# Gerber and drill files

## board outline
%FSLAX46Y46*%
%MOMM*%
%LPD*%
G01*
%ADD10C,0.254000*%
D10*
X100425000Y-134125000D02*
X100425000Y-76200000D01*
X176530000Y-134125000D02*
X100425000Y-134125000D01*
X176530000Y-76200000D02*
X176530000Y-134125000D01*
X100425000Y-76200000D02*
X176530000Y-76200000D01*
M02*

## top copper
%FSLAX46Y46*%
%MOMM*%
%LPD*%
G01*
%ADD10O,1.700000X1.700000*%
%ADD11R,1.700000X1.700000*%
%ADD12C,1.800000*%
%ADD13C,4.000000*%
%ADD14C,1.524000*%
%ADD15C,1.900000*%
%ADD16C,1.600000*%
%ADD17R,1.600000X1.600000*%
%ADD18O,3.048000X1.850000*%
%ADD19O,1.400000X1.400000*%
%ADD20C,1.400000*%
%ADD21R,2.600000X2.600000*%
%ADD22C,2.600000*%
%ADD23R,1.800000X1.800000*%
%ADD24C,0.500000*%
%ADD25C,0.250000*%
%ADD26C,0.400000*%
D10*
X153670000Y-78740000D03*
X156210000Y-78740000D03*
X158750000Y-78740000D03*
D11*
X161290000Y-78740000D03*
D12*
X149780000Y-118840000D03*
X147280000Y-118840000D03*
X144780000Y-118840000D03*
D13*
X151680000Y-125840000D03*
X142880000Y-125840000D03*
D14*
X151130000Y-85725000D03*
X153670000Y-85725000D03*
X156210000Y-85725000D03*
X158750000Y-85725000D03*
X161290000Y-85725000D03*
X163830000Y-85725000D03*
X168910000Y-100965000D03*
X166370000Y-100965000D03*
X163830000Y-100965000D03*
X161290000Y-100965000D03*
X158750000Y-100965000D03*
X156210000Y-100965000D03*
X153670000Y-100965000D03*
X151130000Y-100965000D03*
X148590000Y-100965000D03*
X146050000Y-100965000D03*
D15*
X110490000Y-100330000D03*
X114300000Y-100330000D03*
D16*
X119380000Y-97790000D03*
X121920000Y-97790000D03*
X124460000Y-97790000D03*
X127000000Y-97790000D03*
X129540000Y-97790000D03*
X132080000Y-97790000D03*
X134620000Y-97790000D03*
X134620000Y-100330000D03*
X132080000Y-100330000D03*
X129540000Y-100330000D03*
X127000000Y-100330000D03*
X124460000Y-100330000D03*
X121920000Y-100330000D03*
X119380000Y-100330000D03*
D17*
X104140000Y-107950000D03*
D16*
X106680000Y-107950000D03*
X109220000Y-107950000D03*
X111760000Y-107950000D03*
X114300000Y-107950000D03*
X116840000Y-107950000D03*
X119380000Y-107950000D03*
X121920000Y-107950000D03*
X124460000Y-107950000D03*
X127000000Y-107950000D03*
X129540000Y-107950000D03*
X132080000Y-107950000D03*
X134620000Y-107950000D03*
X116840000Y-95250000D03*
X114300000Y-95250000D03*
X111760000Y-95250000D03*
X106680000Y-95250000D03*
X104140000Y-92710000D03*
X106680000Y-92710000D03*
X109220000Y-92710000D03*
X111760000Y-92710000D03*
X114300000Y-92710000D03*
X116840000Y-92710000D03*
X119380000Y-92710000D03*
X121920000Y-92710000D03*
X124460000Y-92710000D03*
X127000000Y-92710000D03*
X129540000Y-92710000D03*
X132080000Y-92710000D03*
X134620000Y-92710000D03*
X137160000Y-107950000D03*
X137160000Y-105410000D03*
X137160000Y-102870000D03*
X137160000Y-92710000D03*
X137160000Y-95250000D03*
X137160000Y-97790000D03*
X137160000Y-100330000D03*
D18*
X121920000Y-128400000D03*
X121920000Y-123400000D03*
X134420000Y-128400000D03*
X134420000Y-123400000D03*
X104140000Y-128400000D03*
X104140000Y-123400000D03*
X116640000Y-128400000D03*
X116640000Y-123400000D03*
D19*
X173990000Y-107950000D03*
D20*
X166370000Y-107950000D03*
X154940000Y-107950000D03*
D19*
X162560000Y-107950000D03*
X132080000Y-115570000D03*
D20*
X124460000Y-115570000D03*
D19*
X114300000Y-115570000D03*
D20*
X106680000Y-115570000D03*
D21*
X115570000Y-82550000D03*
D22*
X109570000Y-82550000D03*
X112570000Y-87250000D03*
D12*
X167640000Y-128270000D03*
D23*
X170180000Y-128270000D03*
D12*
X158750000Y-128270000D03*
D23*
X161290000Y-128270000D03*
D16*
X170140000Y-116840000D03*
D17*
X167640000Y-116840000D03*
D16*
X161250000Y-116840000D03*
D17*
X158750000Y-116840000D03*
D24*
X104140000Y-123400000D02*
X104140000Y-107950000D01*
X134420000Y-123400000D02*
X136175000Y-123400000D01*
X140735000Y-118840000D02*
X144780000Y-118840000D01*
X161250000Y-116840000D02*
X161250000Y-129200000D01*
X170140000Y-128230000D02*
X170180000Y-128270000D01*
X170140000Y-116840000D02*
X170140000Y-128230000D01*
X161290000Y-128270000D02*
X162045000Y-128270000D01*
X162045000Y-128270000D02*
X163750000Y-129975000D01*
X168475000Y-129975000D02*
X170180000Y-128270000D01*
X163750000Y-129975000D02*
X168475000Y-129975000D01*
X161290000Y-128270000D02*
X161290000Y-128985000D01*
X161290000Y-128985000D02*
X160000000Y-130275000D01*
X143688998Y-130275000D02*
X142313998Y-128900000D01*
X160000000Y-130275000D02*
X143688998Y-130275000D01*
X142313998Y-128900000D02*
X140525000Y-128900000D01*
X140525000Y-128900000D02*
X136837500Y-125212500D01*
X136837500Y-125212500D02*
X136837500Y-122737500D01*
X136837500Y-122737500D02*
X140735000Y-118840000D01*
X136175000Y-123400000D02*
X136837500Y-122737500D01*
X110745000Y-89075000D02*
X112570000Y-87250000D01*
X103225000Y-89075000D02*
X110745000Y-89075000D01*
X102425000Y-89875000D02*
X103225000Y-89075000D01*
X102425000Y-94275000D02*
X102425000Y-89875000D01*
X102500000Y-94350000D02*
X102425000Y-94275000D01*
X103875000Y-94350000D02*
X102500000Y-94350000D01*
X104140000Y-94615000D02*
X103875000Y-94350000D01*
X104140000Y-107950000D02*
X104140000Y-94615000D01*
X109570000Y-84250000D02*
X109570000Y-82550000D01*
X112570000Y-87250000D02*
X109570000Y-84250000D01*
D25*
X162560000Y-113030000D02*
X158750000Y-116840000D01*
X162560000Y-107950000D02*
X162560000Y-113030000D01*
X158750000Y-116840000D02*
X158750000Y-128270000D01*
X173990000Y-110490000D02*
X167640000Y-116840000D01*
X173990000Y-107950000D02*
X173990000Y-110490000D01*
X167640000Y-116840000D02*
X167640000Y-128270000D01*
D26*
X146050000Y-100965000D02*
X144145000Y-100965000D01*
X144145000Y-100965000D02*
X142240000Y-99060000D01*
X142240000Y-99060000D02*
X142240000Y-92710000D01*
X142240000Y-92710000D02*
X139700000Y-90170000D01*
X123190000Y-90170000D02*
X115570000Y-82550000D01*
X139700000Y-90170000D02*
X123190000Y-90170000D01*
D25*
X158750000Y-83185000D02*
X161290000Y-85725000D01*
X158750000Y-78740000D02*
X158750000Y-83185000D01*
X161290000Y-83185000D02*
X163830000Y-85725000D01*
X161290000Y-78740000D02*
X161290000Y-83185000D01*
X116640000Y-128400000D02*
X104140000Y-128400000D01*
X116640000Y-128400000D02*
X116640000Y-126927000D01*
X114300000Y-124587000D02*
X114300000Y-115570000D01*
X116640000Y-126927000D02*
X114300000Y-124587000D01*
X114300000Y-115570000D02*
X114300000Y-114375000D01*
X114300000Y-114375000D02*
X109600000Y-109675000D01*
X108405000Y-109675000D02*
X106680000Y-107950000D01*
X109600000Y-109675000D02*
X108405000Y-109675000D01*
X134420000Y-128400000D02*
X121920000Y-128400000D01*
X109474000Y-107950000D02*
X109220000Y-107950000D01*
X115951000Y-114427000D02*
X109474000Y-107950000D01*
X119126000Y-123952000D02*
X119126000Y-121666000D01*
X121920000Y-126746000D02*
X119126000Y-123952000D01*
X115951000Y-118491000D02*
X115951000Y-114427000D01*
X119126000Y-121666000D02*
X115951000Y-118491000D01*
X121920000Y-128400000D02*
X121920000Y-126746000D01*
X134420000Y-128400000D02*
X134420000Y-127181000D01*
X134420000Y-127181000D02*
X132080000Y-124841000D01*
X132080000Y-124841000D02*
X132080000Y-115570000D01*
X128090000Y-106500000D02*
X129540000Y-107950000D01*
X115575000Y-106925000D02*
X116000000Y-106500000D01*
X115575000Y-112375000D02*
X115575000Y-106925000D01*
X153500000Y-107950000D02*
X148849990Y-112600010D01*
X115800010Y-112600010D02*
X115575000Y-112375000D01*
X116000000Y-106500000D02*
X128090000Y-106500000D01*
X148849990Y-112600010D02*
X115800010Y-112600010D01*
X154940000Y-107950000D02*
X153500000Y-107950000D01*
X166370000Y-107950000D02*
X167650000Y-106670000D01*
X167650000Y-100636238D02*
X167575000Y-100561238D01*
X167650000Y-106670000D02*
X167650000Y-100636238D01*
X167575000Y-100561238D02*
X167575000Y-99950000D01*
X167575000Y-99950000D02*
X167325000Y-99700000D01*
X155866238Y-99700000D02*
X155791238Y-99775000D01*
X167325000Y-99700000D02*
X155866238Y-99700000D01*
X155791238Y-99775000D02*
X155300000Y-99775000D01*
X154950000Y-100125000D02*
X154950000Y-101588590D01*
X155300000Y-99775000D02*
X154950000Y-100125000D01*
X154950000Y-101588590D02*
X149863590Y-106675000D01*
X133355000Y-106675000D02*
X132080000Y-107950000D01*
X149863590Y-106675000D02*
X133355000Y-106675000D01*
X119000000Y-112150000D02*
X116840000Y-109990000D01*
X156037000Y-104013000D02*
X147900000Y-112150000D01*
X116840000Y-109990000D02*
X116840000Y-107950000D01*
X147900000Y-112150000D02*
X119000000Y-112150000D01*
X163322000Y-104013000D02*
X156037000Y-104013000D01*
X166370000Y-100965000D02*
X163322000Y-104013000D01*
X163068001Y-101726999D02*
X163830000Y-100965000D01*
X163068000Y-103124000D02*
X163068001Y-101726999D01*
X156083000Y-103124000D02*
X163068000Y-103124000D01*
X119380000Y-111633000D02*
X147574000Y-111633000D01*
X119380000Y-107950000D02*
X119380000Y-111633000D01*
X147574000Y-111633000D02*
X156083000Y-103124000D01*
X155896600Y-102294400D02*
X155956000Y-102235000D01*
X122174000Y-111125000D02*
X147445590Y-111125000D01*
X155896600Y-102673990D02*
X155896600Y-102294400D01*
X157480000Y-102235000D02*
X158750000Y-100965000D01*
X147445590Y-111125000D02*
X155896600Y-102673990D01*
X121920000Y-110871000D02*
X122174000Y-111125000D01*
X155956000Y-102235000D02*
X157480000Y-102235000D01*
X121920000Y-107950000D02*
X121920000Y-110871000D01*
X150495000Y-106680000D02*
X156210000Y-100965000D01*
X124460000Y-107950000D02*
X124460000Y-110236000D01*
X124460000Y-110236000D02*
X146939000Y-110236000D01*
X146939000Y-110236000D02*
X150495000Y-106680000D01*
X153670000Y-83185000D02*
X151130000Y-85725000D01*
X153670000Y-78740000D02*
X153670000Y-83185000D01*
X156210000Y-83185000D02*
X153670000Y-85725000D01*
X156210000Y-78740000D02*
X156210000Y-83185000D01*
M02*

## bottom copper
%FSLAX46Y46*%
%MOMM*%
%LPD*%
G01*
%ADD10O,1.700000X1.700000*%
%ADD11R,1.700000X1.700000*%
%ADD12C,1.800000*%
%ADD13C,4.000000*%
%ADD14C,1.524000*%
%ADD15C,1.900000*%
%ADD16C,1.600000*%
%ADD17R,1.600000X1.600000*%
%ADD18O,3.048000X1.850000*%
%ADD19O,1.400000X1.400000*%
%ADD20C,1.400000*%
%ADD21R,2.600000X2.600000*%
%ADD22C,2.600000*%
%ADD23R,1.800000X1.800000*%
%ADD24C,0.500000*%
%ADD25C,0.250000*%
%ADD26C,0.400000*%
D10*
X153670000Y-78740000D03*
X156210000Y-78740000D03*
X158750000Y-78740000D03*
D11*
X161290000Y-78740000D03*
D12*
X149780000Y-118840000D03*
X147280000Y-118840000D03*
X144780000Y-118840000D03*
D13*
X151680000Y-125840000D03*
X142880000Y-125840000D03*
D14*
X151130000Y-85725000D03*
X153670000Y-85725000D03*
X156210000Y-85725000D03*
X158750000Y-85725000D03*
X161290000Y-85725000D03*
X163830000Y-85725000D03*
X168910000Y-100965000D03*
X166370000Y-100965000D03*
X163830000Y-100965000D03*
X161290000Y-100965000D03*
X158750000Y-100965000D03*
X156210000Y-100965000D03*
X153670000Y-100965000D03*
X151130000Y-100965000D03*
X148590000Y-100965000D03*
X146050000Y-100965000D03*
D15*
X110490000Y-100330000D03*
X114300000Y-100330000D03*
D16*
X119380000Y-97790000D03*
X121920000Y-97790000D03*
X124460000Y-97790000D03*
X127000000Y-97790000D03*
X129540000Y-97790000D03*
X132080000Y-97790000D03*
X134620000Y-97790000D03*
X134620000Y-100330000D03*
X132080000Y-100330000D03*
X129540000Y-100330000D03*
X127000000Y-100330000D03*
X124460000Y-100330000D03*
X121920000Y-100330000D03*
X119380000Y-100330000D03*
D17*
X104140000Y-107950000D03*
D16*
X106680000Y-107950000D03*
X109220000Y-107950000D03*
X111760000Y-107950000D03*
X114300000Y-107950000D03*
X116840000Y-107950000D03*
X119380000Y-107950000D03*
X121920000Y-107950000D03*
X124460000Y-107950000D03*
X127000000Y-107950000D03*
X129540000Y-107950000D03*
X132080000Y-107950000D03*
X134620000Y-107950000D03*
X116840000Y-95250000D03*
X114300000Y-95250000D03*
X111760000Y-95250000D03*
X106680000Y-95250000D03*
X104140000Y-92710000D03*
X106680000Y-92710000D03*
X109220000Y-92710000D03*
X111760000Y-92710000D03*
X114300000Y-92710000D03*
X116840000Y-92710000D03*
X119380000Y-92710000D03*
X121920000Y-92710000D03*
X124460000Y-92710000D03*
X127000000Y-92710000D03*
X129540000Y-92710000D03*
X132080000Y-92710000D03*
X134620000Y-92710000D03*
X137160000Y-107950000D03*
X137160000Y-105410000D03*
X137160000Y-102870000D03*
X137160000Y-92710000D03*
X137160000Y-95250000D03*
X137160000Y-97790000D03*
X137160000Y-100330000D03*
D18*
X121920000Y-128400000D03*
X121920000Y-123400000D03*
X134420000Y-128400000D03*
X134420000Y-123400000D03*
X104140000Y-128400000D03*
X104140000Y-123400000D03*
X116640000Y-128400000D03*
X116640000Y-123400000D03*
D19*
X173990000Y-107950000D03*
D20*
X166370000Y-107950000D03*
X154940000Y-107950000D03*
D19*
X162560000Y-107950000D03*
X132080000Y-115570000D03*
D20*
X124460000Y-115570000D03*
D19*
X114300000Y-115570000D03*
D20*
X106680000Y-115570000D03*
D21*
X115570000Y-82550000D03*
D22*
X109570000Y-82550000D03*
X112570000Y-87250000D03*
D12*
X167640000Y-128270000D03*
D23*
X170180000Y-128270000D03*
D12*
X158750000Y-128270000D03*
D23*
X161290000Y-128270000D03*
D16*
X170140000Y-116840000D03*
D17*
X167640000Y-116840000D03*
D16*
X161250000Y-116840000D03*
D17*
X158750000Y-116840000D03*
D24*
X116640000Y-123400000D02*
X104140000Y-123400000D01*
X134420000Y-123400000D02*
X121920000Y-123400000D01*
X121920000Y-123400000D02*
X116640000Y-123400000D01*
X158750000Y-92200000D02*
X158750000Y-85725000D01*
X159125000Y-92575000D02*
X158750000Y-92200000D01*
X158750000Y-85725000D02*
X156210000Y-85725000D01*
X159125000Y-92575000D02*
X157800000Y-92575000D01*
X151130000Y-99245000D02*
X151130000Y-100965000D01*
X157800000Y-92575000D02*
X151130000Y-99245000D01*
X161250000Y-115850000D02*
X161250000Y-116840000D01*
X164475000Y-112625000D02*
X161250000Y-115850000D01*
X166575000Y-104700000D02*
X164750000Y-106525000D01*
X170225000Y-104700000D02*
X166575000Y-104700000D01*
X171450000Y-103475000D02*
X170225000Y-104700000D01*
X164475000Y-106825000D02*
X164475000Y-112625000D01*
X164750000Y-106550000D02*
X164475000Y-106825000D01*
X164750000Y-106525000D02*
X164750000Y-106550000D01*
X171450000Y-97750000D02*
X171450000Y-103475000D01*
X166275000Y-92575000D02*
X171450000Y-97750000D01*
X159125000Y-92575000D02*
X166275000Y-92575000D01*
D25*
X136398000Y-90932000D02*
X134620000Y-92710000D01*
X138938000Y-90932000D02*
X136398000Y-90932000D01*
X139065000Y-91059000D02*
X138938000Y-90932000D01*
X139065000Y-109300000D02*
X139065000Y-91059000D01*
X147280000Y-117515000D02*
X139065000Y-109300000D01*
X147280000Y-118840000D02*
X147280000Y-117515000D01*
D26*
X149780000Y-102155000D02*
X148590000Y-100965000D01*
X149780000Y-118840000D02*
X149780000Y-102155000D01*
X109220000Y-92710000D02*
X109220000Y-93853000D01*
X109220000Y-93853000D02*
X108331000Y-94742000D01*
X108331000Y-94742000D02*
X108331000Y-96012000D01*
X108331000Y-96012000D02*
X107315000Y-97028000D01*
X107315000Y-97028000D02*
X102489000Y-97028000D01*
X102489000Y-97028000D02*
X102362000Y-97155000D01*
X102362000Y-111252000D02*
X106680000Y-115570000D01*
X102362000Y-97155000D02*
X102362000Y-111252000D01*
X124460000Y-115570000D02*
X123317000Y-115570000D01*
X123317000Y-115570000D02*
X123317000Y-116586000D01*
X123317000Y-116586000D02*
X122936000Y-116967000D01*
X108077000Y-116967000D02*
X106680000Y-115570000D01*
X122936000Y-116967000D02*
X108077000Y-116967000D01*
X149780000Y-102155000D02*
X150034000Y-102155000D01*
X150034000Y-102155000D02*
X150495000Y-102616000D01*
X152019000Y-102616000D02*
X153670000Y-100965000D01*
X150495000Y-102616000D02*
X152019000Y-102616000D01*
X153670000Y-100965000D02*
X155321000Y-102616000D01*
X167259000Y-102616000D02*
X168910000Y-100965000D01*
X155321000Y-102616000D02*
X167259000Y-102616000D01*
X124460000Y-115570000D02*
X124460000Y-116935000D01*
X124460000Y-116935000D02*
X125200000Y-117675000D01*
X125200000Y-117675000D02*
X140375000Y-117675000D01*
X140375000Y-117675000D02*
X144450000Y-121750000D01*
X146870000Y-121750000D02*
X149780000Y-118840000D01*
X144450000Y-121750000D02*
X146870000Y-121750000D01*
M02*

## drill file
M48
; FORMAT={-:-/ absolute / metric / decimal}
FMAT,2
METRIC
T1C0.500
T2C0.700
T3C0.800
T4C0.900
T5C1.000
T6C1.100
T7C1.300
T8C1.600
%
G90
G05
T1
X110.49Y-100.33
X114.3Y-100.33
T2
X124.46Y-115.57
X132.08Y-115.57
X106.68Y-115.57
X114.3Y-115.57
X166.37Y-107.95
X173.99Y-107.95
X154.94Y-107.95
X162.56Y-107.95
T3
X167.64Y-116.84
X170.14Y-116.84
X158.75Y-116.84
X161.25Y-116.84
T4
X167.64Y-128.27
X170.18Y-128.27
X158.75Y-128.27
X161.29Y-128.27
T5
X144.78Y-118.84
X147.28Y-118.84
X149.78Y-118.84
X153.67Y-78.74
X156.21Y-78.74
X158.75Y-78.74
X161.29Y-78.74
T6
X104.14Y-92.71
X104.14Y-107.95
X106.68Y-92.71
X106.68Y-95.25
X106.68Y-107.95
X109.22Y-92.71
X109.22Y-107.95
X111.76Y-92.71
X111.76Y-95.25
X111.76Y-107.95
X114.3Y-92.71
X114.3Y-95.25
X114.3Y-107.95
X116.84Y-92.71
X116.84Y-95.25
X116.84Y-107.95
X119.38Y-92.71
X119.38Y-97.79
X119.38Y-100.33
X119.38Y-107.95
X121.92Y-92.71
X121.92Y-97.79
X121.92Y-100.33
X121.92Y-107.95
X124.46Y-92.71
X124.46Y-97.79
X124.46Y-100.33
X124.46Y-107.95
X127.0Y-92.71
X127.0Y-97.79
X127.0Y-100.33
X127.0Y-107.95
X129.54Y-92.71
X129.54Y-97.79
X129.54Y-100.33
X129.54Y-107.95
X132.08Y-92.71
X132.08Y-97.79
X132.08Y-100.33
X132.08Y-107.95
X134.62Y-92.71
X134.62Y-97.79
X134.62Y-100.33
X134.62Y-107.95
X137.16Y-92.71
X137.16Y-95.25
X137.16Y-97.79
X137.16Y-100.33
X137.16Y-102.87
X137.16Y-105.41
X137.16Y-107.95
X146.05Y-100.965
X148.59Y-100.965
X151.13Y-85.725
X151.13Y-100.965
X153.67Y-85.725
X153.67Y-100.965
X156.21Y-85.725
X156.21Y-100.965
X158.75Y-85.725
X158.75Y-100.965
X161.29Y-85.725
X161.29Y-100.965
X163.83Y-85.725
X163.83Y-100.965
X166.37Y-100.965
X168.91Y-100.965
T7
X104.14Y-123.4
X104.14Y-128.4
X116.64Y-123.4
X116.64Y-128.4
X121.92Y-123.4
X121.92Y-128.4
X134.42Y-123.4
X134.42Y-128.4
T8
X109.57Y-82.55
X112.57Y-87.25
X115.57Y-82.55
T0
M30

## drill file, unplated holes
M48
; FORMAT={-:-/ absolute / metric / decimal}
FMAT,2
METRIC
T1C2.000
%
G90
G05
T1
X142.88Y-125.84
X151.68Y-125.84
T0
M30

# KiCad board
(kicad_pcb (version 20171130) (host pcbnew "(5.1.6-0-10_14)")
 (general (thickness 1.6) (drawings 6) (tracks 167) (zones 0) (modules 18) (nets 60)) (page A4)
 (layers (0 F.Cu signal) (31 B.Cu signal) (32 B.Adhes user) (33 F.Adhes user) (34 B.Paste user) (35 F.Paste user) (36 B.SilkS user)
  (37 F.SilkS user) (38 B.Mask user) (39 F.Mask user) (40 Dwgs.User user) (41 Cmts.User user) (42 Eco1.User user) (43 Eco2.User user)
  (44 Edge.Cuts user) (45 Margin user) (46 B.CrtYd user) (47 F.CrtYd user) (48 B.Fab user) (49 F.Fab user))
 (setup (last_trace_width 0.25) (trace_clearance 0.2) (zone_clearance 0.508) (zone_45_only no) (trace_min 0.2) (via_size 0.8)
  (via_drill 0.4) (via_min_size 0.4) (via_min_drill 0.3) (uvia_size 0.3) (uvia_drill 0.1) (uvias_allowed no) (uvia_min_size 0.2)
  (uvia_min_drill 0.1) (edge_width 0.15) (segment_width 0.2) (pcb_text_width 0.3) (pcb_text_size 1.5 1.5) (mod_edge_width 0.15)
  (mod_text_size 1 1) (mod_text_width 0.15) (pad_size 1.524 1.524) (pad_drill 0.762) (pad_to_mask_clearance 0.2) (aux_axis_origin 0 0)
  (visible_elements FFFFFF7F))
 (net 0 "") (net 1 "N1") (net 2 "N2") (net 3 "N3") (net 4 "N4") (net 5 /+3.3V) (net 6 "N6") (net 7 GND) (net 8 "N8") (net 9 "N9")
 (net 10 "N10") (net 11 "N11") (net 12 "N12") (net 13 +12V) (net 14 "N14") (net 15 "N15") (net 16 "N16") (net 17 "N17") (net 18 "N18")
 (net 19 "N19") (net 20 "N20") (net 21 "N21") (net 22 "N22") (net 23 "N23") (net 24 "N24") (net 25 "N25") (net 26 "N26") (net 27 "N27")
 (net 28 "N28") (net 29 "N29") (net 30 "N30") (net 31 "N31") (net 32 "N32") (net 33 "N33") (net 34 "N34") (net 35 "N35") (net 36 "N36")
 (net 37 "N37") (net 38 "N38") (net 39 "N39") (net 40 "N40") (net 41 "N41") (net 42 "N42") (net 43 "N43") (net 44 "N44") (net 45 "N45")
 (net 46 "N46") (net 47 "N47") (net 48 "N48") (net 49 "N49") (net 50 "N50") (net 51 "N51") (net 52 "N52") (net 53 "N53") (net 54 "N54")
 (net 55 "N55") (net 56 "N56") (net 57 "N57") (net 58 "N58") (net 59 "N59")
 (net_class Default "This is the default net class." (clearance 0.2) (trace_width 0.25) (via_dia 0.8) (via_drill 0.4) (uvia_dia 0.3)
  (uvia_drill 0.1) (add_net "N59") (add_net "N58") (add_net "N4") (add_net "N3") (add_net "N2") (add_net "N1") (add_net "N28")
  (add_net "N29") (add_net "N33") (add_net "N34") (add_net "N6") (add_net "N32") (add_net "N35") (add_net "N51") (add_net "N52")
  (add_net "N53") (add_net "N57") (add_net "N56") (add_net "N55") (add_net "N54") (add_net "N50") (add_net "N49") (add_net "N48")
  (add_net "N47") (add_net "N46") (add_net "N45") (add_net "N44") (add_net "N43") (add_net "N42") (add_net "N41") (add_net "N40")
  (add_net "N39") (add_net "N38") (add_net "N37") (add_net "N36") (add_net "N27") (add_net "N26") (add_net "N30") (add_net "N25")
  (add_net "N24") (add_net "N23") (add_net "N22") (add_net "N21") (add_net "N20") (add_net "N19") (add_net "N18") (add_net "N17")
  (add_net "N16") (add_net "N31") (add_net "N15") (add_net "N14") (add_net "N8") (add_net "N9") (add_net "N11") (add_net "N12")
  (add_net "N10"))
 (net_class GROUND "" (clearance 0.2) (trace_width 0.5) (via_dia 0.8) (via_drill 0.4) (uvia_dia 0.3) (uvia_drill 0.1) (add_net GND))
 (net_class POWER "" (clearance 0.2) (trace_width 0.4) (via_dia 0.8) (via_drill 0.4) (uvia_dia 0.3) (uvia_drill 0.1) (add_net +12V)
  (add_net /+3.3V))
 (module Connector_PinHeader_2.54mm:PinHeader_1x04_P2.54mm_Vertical (layer F.Cu) (at 161.29 78.74 270)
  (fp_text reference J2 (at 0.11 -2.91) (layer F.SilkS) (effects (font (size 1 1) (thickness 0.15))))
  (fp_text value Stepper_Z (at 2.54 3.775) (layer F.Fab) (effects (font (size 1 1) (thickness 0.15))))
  (pad 4 thru_hole oval (at 0 7.62 270) (size 1.7 1.7) (drill 1) (layers *.Cu *.Mask) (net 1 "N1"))
  (pad 3 thru_hole oval (at 0 5.08 270) (size 1.7 1.7) (drill 1) (layers *.Cu *.Mask) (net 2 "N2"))
  (pad 2 thru_hole oval (at 0 2.54 270) (size 1.7 1.7) (drill 1) (layers *.Cu *.Mask) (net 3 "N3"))
  (pad 1 thru_hole rect (at 0 0 270) (size 1.7 1.7) (drill 1) (layers *.Cu *.Mask) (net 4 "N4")))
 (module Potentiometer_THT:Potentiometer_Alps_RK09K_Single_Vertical (layer F.Cu) (at 144.78 118.84 270)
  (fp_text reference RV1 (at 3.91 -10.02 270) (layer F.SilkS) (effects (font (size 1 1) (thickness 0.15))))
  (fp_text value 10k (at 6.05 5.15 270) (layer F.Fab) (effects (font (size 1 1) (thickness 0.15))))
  (pad 3 thru_hole circle (at 0 -5 270) (size 1.8 1.8) (drill 1) (layers *.Cu *.Mask) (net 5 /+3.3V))
  (pad 2 thru_hole circle (at 0 -2.5 270) (size 1.8 1.8) (drill 1) (layers *.Cu *.Mask) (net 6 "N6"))
  (pad 1 thru_hole circle (at 0 0 270) (size 1.8 1.8) (drill 1) (layers *.Cu *.Mask) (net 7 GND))
  (pad "" np_thru_hole circle (at 7 -6.9 270) (size 4 4) (drill 2) (layers *.Cu *.Mask))
  (pad "" np_thru_hole circle (at 7 1.9 270) (size 4 4) (drill 2) (layers *.Cu *.Mask)))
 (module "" (layer F.Cu) (at 149.86 129.54)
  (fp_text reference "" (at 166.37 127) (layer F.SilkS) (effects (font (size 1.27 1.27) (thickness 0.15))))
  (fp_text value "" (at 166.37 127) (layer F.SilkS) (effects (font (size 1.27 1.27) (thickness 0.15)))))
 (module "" (layer F.Cu) (at 166.37 127)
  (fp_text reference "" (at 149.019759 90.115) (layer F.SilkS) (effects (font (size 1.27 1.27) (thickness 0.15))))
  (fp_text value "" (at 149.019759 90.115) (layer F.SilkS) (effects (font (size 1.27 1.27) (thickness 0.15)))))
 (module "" (layer F.Cu) (at 148.59 127)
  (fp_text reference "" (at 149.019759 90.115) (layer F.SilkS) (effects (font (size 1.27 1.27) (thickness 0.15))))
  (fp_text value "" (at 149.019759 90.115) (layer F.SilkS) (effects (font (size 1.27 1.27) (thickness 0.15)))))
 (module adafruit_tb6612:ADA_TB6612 (layer F.Cu) (at 157.48 93.98 90)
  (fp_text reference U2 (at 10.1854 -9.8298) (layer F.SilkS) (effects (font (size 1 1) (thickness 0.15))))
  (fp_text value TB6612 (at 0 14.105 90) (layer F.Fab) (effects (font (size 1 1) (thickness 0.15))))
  (pad 16 thru_hole circle (at 8.255 -6.35 90) (size 1.524 1.524) (drill 1.1) (layers *.Cu *.Mask) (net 1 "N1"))
  (pad 15 thru_hole circle (at 8.255 -3.81 90) (size 1.524 1.524) (drill 1.1) (layers *.Cu *.Mask) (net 2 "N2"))
  (pad 14 thru_hole circle (at 8.255 -1.27 90) (size 1.524 1.524) (drill 1.1) (layers *.Cu *.Mask) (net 7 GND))
  (pad 13 thru_hole circle (at 8.255 1.27 90) (size 1.524 1.524) (drill 1.1) (layers *.Cu *.Mask) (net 7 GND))
  (pad 12 thru_hole circle (at 8.255 3.81 90) (size 1.524 1.524) (drill 1.1) (layers *.Cu *.Mask) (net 3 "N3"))
  (pad 11 thru_hole circle (at 8.255 6.35 90) (size 1.524 1.524) (drill 1.1) (layers *.Cu *.Mask) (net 4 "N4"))
  (pad 10 thru_hole circle (at -6.985 11.43 90) (size 1.524 1.524) (drill 1.1) (layers *.Cu *.Mask) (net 5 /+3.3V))
  (pad 9 thru_hole circle (at -6.985 8.89 90) (size 1.524 1.524) (drill 1.1) (layers *.Cu *.Mask) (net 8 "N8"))
  (pad 8 thru_hole circle (at -6.985 6.35 90) (size 1.524 1.524) (drill 1.1) (layers *.Cu *.Mask) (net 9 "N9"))
  (pad 7 thru_hole circle (at -6.985 3.81 90) (size 1.524 1.524) (drill 1.1) (layers *.Cu *.Mask) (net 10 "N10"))
  (pad 6 thru_hole circle (at -6.985 1.27 90) (size 1.524 1.524) (drill 1.1) (layers *.Cu *.Mask) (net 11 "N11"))
  (pad 5 thru_hole circle (at -6.985 -1.27 90) (size 1.524 1.524) (drill 1.1) (layers *.Cu *.Mask) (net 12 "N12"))
  (pad 4 thru_hole circle (at -6.985 -3.81 90) (size 1.524 1.524) (drill 1.1) (layers *.Cu *.Mask) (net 5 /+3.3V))
  (pad 3 thru_hole circle (at -6.985 -6.35 90) (size 1.524 1.524) (drill 1.1) (layers *.Cu *.Mask) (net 7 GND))
  (pad 2 thru_hole circle (at -6.985 -8.89 90) (size 1.524 1.524) (drill 1.1) (layers *.Cu *.Mask) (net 5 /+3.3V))
  (pad 1 thru_hole circle (at -6.985 -11.43 90) (size 1.524 1.524) (drill 1.1) (layers *.Cu *.Mask) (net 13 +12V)))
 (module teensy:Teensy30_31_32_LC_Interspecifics (layer F.Cu) (at 120.65 100.33)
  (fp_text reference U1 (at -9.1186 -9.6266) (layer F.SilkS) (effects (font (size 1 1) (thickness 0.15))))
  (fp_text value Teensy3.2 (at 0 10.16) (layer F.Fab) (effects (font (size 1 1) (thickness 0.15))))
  (pad 52 thru_hole circle (at -10.16 0) (size 1.9 1.9) (drill 0.5) (layers *.Cu *.Mask F.SilkS))
  (pad 52 thru_hole circle (at -6.35 0) (size 1.9 1.9) (drill 0.5) (layers *.Cu *.Mask F.SilkS))
  (pad 51 thru_hole circle (at -1.27 -2.54) (size 1.6 1.6) (drill 1.1) (layers *.Cu *.Mask) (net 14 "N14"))
  (pad 50 thru_hole circle (at 1.27 -2.54) (size 1.6 1.6) (drill 1.1) (layers *.Cu *.Mask) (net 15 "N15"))
  (pad 49 thru_hole circle (at 3.81 -2.54) (size 1.6 1.6) (drill 1.1) (layers *.Cu *.Mask) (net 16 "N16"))
  (pad 48 thru_hole circle (at 6.35 -2.54) (size 1.6 1.6) (drill 1.1) (layers *.Cu *.Mask) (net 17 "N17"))
  (pad 47 thru_hole circle (at 8.89 -2.54) (size 1.6 1.6) (drill 1.1) (layers *.Cu *.Mask) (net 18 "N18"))
  (pad 46 thru_hole circle (at 11.43 -2.54) (size 1.6 1.6) (drill 1.1) (layers *.Cu *.Mask) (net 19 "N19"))
  (pad 45 thru_hole circle (at 13.97 -2.54) (size 1.6 1.6) (drill 1.1) (layers *.Cu *.Mask) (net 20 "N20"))
  (pad 44 thru_hole circle (at 13.97 0) (size 1.6 1.6) (drill 1.1) (layers *.Cu *.Mask) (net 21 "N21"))
  (pad 43 thru_hole circle (at 11.43 0) (size 1.6 1.6) (drill 1.1) (layers *.Cu *.Mask) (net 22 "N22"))
  (pad 42 thru_hole circle (at 8.89 0) (size 1.6 1.6) (drill 1.1) (layers *.Cu *.Mask) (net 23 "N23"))
  (pad 41 thru_hole circle (at 6.35 0) (size 1.6 1.6) (drill 1.1) (layers *.Cu *.Mask) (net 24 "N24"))
  (pad 40 thru_hole circle (at 3.81 0) (size 1.6 1.6) (drill 1.1) (layers *.Cu *.Mask) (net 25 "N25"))
  (pad 39 thru_hole circle (at 1.27 0) (size 1.6 1.6) (drill 1.1) (layers *.Cu *.Mask) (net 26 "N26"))
  (pad 38 thru_hole circle (at -1.27 0) (size 1.6 1.6) (drill 1.1) (layers *.Cu *.Mask) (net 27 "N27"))
  (pad 1 thru_hole rect (at -16.51 7.62) (size 1.6 1.6) (drill 1.1) (layers *.Cu *.Mask F.SilkS) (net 7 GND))
  (pad 2 thru_hole circle (at -13.97 7.62) (size 1.6 1.6) (drill 1.1) (layers *.Cu *.Mask F.SilkS) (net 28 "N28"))
  (pad 3 thru_hole circle (at -11.43 7.62) (size 1.6 1.6) (drill 1.1) (layers *.Cu *.Mask F.SilkS) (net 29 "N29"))
  (pad 4 thru_hole circle (at -8.89 7.62) (size 1.6 1.6) (drill 1.1) (layers *.Cu *.Mask F.SilkS) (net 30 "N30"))
  (pad 5 thru_hole circle (at -6.35 7.62) (size 1.6 1.6) (drill 1.1) (layers *.Cu *.Mask F.SilkS) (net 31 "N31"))
  (pad 6 thru_hole circle (at -3.81 7.62) (size 1.6 1.6) (drill 1.1) (layers *.Cu *.Mask F.SilkS) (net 8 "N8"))
  (pad 7 thru_hole circle (at -1.27 7.62) (size 1.6 1.6) (drill 1.1) (layers *.Cu *.Mask F.SilkS) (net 9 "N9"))
  (pad 8 thru_hole circle (at 1.27 7.62) (size 1.6 1.6) (drill 1.1) (layers *.Cu *.Mask F.SilkS) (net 11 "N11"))
  (pad 9 thru_hole circle (at 3.81 7.62) (size 1.6 1.6) (drill 1.1) (layers *.Cu *.Mask F.SilkS) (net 12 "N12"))
  (pad 10 thru_hole circle (at 6.35 7.62) (size 1.6 1.6) (drill 1.1) (layers *.Cu *.Mask F.SilkS) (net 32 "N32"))
  (pad 11 thru_hole circle (at 8.89 7.62) (size 1.6 1.6) (drill 1.1) (layers *.Cu *.Mask F.SilkS) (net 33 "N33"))
  (pad 12 thru_hole circle (at 11.43 7.62) (size 1.6 1.6) (drill 1.1) (layers *.Cu *.Mask F.SilkS) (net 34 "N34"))
  (pad 13 thru_hole circle (at 13.97 7.62) (size 1.6 1.6) (drill 1.1) (layers *.Cu *.Mask F.SilkS) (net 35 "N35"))
  (pad 37 thru_hole circle (at -3.81 -5.08) (size 1.6 1.6) (drill 1.1) (layers *.Cu *.Mask F.SilkS) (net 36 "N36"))
  (pad 36 thru_hole circle (at -6.35 -5.08) (size 1.6 1.6) (drill 1.1) (layers *.Cu *.Mask F.SilkS) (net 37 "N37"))
  (pad 35 thru_hole circle (at -8.89 -5.08) (size 1.6 1.6) (drill 1.1) (layers *.Cu *.Mask F.SilkS) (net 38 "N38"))
  (pad 34 thru_hole circle (at -13.97 -5.08) (size 1.6 1.6) (drill 1.1) (layers *.Cu *.Mask F.SilkS) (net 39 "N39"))
  (pad 33 thru_hole circle (at -16.51 -7.62) (size 1.6 1.6) (drill 1.1) (layers *.Cu *.Mask F.SilkS) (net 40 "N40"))
  (pad 32 thru_hole circle (at -13.97 -7.62) (size 1.6 1.6) (drill 1.1) (layers *.Cu *.Mask F.SilkS) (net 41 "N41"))
  (pad 31 thru_hole circle (at -11.43 -7.62) (size 1.6 1.6) (drill 1.1) (layers *.Cu *.Mask F.SilkS) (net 5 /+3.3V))
  (pad 30 thru_hole circle (at -8.89 -7.62) (size 1.6 1.6) (drill 1.1) (layers *.Cu *.Mask F.SilkS) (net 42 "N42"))
  (pad 29 thru_hole circle (at -6.35 -7.62) (size 1.6 1.6) (drill 1.1) (layers *.Cu *.Mask F.SilkS) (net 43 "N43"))
  (pad 28 thru_hole circle (at -3.81 -7.62) (size 1.6 1.6) (drill 1.1) (layers *.Cu *.Mask F.SilkS) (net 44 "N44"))
  (pad 27 thru_hole circle (at -1.27 -7.62) (size 1.6 1.6) (drill 1.1) (layers *.Cu *.Mask F.SilkS) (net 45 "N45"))
  (pad 26 thru_hole circle (at 1.27 -7.62) (size 1.6 1.6) (drill 1.1) (layers *.Cu *.Mask F.SilkS) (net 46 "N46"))
  (pad 25 thru_hole circle (at 3.81 -7.62) (size 1.6 1.6) (drill 1.1) (layers *.Cu *.Mask F.SilkS) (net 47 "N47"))
  (pad 24 thru_hole circle (at 6.35 -7.62) (size 1.6 1.6) (drill 1.1) (layers *.Cu *.Mask F.SilkS) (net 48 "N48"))
  (pad 23 thru_hole circle (at 8.89 -7.62) (size 1.6 1.6) (drill 1.1) (layers *.Cu *.Mask F.SilkS) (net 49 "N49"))
  (pad 22 thru_hole circle (at 11.43 -7.62) (size 1.6 1.6) (drill 1.1) (layers *.Cu *.Mask F.SilkS) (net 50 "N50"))
  (pad 21 thru_hole circle (at 13.97 -7.62) (size 1.6 1.6) (drill 1.1) (layers *.Cu *.Mask F.SilkS) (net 6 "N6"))
  (pad 14 thru_hole circle (at 16.51 7.62) (size 1.6 1.6) (drill 1.1) (layers *.Cu *.Mask F.SilkS) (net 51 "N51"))
  (pad 15 thru_hole circle (at 16.51 5.08) (size 1.6 1.6) (drill 1.1) (layers *.Cu *.Mask F.SilkS) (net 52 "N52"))
  (pad 16 thru_hole circle (at 16.51 2.54) (size 1.6 1.6) (drill 1.1) (layers *.Cu *.Mask F.SilkS) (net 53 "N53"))
  (pad 20 thru_hole circle (at 16.51 -7.62) (size 1.6 1.6) (drill 1.1) (layers *.Cu *.Mask F.SilkS) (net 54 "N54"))
  (pad 19 thru_hole circle (at 16.51 -5.08) (size 1.6 1.6) (drill 1.1) (layers *.Cu *.Mask F.SilkS) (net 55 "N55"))
  (pad 18 thru_hole circle (at 16.51 -2.54) (size 1.6 1.6) (drill 1.1) (layers *.Cu *.Mask F.SilkS) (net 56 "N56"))
  (pad 17 thru_hole circle (at 16.51 0) (size 1.6 1.6) (drill 1.1) (layers *.Cu *.Mask F.SilkS) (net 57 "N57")))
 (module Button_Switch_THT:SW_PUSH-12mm (layer F.Cu) (at 121.92 123.4)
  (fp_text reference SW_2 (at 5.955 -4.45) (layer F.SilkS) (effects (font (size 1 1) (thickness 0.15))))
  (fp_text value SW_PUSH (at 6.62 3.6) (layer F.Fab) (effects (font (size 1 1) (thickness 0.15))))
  (pad 2 thru_hole oval (at 0 5) (size 3.048 1.85) (drill 1.3) (layers *.Cu *.Mask) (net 29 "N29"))
  (pad 1 thru_hole oval (at 0 0) (size 3.048 1.85) (drill 1.3) (layers *.Cu *.Mask) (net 7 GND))
  (pad 2 thru_hole oval (at 12.5 5) (size 3.048 1.85) (drill 1.3) (layers *.Cu *.Mask) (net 29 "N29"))
  (pad 1 thru_hole oval (at 12.5 0) (size 3.048 1.85) (drill 1.3) (layers *.Cu *.Mask) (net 7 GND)))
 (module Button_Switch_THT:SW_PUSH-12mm (layer F.Cu) (at 104.14 123.4)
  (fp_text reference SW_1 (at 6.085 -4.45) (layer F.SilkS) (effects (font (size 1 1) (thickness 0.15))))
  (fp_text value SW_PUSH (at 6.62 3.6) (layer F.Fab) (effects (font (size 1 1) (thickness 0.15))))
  (pad 2 thru_hole oval (at 0 5) (size 3.048 1.85) (drill 1.3) (layers *.Cu *.Mask) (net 28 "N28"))
  (pad 1 thru_hole oval (at 0 0) (size 3.048 1.85) (drill 1.3) (layers *.Cu *.Mask) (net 7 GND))
  (pad 2 thru_hole oval (at 12.5 5) (size 3.048 1.85) (drill 1.3) (layers *.Cu *.Mask) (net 28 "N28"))
  (pad 1 thru_hole oval (at 12.5 0) (size 3.048 1.85) (drill 1.3) (layers *.Cu *.Mask) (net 7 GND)))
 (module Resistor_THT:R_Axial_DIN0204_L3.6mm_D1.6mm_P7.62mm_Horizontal (layer F.Cu) (at 166.37 107.95)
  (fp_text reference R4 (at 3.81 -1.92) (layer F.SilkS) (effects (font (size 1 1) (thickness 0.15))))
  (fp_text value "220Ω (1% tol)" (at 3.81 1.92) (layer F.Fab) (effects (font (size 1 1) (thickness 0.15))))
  (pad 2 thru_hole oval (at 7.62 0) (size 1.4 1.4) (drill 0.7) (layers *.Cu *.Mask) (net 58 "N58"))
  (pad 1 thru_hole circle (at 0 0) (size 1.4 1.4) (drill 0.7) (layers *.Cu *.Mask) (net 34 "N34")))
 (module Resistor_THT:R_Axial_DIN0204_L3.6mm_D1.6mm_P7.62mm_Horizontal (layer F.Cu) (at 154.94 107.95)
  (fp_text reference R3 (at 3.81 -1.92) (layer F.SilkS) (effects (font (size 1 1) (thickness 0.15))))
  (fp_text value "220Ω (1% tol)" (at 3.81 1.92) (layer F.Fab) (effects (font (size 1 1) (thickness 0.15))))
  (pad 1 thru_hole circle (at 0 0) (size 1.4 1.4) (drill 0.7) (layers *.Cu *.Mask) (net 33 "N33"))
  (pad 2 thru_hole oval (at 7.62 0) (size 1.4 1.4) (drill 0.7) (layers *.Cu *.Mask) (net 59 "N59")))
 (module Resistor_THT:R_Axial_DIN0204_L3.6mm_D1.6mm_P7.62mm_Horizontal (layer F.Cu) (at 124.46 115.57)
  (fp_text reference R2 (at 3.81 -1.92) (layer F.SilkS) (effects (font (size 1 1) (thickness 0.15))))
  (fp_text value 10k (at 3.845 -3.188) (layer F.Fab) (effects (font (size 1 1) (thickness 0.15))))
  (pad 2 thru_hole oval (at 7.62 0) (size 1.4 1.4) (drill 0.7) (layers *.Cu *.Mask) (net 29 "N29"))
  (pad 1 thru_hole circle (at 0 0) (size 1.4 1.4) (drill 0.7) (layers *.Cu *.Mask) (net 5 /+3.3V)))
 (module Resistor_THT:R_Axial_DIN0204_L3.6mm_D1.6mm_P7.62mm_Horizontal (layer F.Cu) (at 106.68 115.57)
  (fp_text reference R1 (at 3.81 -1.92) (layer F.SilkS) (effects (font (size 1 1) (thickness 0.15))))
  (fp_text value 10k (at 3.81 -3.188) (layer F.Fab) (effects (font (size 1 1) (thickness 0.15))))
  (pad 2 thru_hole oval (at 7.62 0) (size 1.4 1.4) (drill 0.7) (layers *.Cu *.Mask) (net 28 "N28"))
  (pad 1 thru_hole circle (at 0 0) (size 1.4 1.4) (drill 0.7) (layers *.Cu *.Mask) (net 5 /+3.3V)))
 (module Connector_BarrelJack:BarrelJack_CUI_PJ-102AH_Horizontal (layer F.Cu) (at 115.57 82.55 270)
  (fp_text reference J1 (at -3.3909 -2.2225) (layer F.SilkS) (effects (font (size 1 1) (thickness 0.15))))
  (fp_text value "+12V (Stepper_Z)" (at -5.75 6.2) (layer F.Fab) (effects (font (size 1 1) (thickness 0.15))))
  (pad 1 thru_hole rect (at 0 0 270) (size 2.6 2.6) (drill 1.6) (layers *.Cu *.Mask) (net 13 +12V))
  (pad 2 thru_hole circle (at 0 6 270) (size 2.6 2.6) (drill 1.6) (layers *.Cu *.Mask) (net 7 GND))
  (pad 3 thru_hole circle (at 4.7 3 270) (size 2.6 2.6) (drill 1.6) (layers *.Cu *.Mask) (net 7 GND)))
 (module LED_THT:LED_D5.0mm (layer F.Cu) (at 170.18 128.27 180)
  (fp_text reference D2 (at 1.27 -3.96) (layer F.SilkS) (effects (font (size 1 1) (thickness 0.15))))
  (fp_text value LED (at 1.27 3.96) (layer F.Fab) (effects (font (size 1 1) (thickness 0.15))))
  (pad 2 thru_hole circle (at 2.54 0 180) (size 1.8 1.8) (drill 0.9) (layers *.Cu *.Mask) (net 58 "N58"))
  (pad 1 thru_hole rect (at 0 0 180) (size 1.8 1.8) (drill 0.9) (layers *.Cu *.Mask) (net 7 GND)))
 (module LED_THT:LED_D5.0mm (layer F.Cu) (at 161.29 128.27 180)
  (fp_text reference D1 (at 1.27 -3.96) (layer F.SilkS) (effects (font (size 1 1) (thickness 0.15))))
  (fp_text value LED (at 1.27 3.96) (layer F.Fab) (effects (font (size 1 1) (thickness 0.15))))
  (pad 2 thru_hole circle (at 2.54 0 180) (size 1.8 1.8) (drill 0.9) (layers *.Cu *.Mask) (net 59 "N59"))
  (pad 1 thru_hole rect (at 0 0 180) (size 1.8 1.8) (drill 0.9) (layers *.Cu *.Mask) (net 7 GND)))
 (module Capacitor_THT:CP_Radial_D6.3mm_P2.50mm (layer F.Cu) (at 167.64 116.84)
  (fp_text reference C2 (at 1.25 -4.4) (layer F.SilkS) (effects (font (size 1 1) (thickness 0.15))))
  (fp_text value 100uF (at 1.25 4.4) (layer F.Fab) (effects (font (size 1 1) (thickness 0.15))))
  (pad 2 thru_hole circle (at 2.5 0) (size 1.6 1.6) (drill 0.8) (layers *.Cu *.Mask) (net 7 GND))
  (pad 1 thru_hole rect (at 0 0) (size 1.6 1.6) (drill 0.8) (layers *.Cu *.Mask) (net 58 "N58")))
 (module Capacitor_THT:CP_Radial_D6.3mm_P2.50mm (layer F.Cu) (at 158.75 116.84)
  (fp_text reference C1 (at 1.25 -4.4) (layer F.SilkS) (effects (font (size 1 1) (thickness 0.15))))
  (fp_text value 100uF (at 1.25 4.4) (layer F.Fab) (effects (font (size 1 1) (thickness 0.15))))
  (pad 2 thru_hole circle (at 2.5 0) (size 1.6 1.6) (drill 0.8) (layers *.Cu *.Mask) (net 7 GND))
  (pad 1 thru_hole rect (at 0 0) (size 1.6 1.6) (drill 0.8) (layers *.Cu *.Mask) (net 59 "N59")))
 (gr_line (start 100.425 134.125) (end 100.425 76.2) (layer Edge.Cuts) (width 0.254))
 (gr_line (start 176.53 134.125) (end 100.425 134.125) (layer Edge.Cuts) (width 0.254))
 (gr_line (start 176.53 76.2) (end 176.53 134.125) (layer Edge.Cuts) (width 0.254))
 (gr_line (start 100.425 76.2) (end 176.53 76.2) (layer Edge.Cuts) (width 0.254))
 (segment (start 104.14 123.4) (end 104.14 107.95) (width 0.5) (layer F.Cu) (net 7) (status 30))
 (segment (start 116.64 123.4) (end 104.14 123.4) (width 0.5) (layer B.Cu) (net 7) (status 30))
 (segment (start 134.42 123.4) (end 121.92 123.4) (width 0.5) (layer B.Cu) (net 7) (status 30))
 (segment (start 121.92 123.4) (end 116.64 123.4) (width 0.5) (layer B.Cu) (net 7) (status 30))
 (segment (start 134.42 123.4) (end 136.175 123.4) (width 0.5) (layer F.Cu) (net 7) (status 10))
 (segment (start 140.735 118.84) (end 144.78 118.84) (width 0.5) (layer F.Cu) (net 7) (status 20))
 (segment (start 161.25 116.84) (end 161.25 129.2) (width 0.5) (layer F.Cu) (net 7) (status 10))
 (segment (start 170.14 128.23) (end 170.18 128.27) (width 0.5) (layer F.Cu) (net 7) (status 30))
 (segment (start 170.14 116.84) (end 170.14 128.23) (width 0.5) (layer F.Cu) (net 7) (status 30))
 (segment (start 161.29 128.27) (end 162.045 128.27) (width 0.5) (layer F.Cu) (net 7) (status 30))
 (segment (start 162.045 128.27) (end 163.75 129.975) (width 0.5) (layer F.Cu) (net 7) (status 10))
 (segment (start 168.475 129.975) (end 170.18 128.27) (width 0.5) (layer F.Cu) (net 7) (status 20))
 (segment (start 163.75 129.975) (end 168.475 129.975) (width 0.5) (layer F.Cu) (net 7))
 (segment (start 158.75 92.2) (end 158.75 85.725) (width 0.5) (layer B.Cu) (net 7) (status 20))
 (segment (start 159.125 92.575) (end 158.75 92.2) (width 0.5) (layer B.Cu) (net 7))
 (segment (start 158.75 85.725) (end 156.21 85.725) (width 0.5) (layer B.Cu) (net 7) (status 30))
 (segment (start 159.125 92.575) (end 157.8 92.575) (width 0.5) (layer B.Cu) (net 7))
 (segment (start 151.13 99.245) (end 151.13 100.965) (width 0.5) (layer B.Cu) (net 7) (status 20))
 (segment (start 157.8 92.575) (end 151.13 99.245) (width 0.5) (layer B.Cu) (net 7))
 (segment (start 161.29 128.27) (end 161.29 128.985) (width 0.5) (layer F.Cu) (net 7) (status 30))
 (segment (start 161.29 128.985) (end 160 130.275) (width 0.5) (layer F.Cu) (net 7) (status 10))
 (segment (start 143.688998 130.275) (end 142.313998 128.9) (width 0.5) (layer F.Cu) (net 7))
 (segment (start 160 130.275) (end 143.688998 130.275) (width 0.5) (layer F.Cu) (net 7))
 (segment (start 142.313998 128.9) (end 140.525 128.9) (width 0.5) (layer F.Cu) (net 7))
 (segment (start 140.525 128.9) (end 136.8375 125.2125) (width 0.5) (layer F.Cu) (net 7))
 (segment (start 136.8375 125.2125) (end 136.8375 122.7375) (width 0.5) (layer F.Cu) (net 7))
 (segment (start 136.8375 122.7375) (end 140.735 118.84) (width 0.5) (layer F.Cu) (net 7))
 (segment (start 136.175 123.4) (end 136.8375 122.7375) (width 0.5) (layer F.Cu) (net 7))
 (segment (start 110.745 89.075) (end 112.57 87.25) (width 0.5) (layer F.Cu) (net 7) (status 20))
 (segment (start 103.225 89.075) (end 110.745 89.075) (width 0.5) (layer F.Cu) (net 7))
 (segment (start 102.425 89.875) (end 103.225 89.075) (width 0.5) (layer F.Cu) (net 7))
 (segment (start 102.425 94.275) (end 102.425 89.875) (width 0.5) (layer F.Cu) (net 7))
 (segment (start 102.5 94.35) (end 102.425 94.275) (width 0.5) (layer F.Cu) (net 7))
 (segment (start 103.875 94.35) (end 102.5 94.35) (width 0.5) (layer F.Cu) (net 7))
 (segment (start 104.14 94.615) (end 103.875 94.35) (width 0.5) (layer F.Cu) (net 7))
 (segment (start 104.14 107.95) (end 104.14 94.615) (width 0.5) (layer F.Cu) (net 7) (status 10))
 (segment (start 109.57 84.25) (end 109.57 82.55) (width 0.5) (layer F.Cu) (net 7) (status 20))
 (segment (start 112.57 87.25) (end 109.57 84.25) (width 0.5) (layer F.Cu) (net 7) (status 10))
 (segment (start 161.25 115.85) (end 161.25 116.84) (width 0.5) (layer B.Cu) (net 7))
 (segment (start 164.475 112.625) (end 161.25 115.85) (width 0.5) (layer B.Cu) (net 7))
 (segment (start 166.575 104.7) (end 164.75 106.525) (width 0.5) (layer B.Cu) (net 7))
 (segment (start 170.225 104.7) (end 166.575 104.7) (width 0.5) (layer B.Cu) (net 7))
 (segment (start 171.45 103.475) (end 170.225 104.7) (width 0.5) (layer B.Cu) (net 7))
 (segment (start 164.475 106.825) (end 164.475 112.625) (width 0.5) (layer B.Cu) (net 7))
 (segment (start 164.75 106.55) (end 164.475 106.825) (width 0.5) (layer B.Cu) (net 7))
 (segment (start 164.75 106.525) (end 164.75 106.55) (width 0.5) (layer B.Cu) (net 7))
 (segment (start 171.45 97.75) (end 171.45 103.475) (width 0.5) (layer B.Cu) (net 7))
 (segment (start 166.275 92.575) (end 171.45 97.75) (width 0.5) (layer B.Cu) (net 7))
 (segment (start 159.125 92.575) (end 166.275 92.575) (width 0.5) (layer B.Cu) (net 7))
 (segment (start 162.56 113.03) (end 158.75 116.84) (width 0.25) (layer F.Cu) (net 59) (status 20))
 (segment (start 162.56 107.95) (end 162.56 113.03) (width 0.25) (layer F.Cu) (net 59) (status 10))
 (segment (start 158.75 116.84) (end 158.75 128.27) (width 0.25) (layer F.Cu) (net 59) (status 30))
 (segment (start 173.99 110.49) (end 167.64 116.84) (width 0.25) (layer F.Cu) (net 58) (status 20))
 (segment (start 173.99 107.95) (end 173.99 110.49) (width 0.25) (layer F.Cu) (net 58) (status 10))
 (segment (start 167.64 116.84) (end 167.64 128.27) (width 0.25) (layer F.Cu) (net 58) (status 30))
 (segment (start 146.05 100.965) (end 144.145 100.965) (width 0.4) (layer F.Cu) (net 13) (status 10))
 (segment (start 144.145 100.965) (end 142.24 99.06) (width 0.4) (layer F.Cu) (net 13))
 (segment (start 142.24 99.06) (end 142.24 92.71) (width 0.4) (layer F.Cu) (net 13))
 (segment (start 142.24 92.71) (end 139.7 90.17) (width 0.4) (layer F.Cu) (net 13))
 (segment (start 123.19 90.17) (end 115.57 82.55) (width 0.4) (layer F.Cu) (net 13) (status 20))
 (segment (start 139.7 90.17) (end 123.19 90.17) (width 0.4) (layer F.Cu) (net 13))
 (segment (start 158.75 83.185) (end 161.29 85.725) (width 0.25) (layer F.Cu) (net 3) (status 20))
 (segment (start 158.75 78.74) (end 158.75 83.185) (width 0.25) (layer F.Cu) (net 3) (status 10))
 (segment (start 161.29 83.185) (end 163.83 85.725) (width 0.25) (layer F.Cu) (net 4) (status 20))
 (segment (start 161.29 78.74) (end 161.29 83.185) (width 0.25) (layer F.Cu) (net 4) (status 10))
 (segment (start 116.64 128.4) (end 104.14 128.4) (width 0.25) (layer F.Cu) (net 28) (status 30))
 (segment (start 116.64 128.4) (end 116.64 126.927) (width 0.25) (layer F.Cu) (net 28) (status 10))
 (segment (start 114.3 124.587) (end 114.3 115.57) (width 0.25) (layer F.Cu) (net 28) (status 20))
 (segment (start 116.64 126.927) (end 114.3 124.587) (width 0.25) (layer F.Cu) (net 28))
 (segment (start 114.3 115.57) (end 114.3 114.375) (width 0.25) (layer F.Cu) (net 28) (status 10))
 (segment (start 114.3 114.375) (end 109.6 109.675) (width 0.25) (layer F.Cu) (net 28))
 (segment (start 108.405 109.675) (end 106.68 107.95) (width 0.25) (layer F.Cu) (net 28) (status 20))
 (segment (start 109.6 109.675) (end 108.405 109.675) (width 0.25) (layer F.Cu) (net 28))
 (segment (start 134.42 128.4) (end 121.92 128.4) (width 0.25) (layer F.Cu) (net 29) (status 30))
 (segment (start 109.474 107.95) (end 109.22 107.95) (width 0.25) (layer F.Cu) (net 29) (status 30))
 (segment (start 115.951 114.427) (end 109.474 107.95) (width 0.25) (layer F.Cu) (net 29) (status 20))
 (segment (start 119.126 123.952) (end 119.126 121.666) (width 0.25) (layer F.Cu) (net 29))
 (segment (start 121.92 126.746) (end 119.126 123.952) (width 0.25) (layer F.Cu) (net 29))
 (segment (start 115.951 118.491) (end 115.951 114.427) (width 0.25) (layer F.Cu) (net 29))
 (segment (start 119.126 121.666) (end 115.951 118.491) (width 0.25) (layer F.Cu) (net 29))
 (segment (start 121.92 128.4) (end 121.92 126.746) (width 0.25) (layer F.Cu) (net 29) (status 10))
 (segment (start 134.42 128.4) (end 134.42 127.181) (width 0.25) (layer F.Cu) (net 29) (status 10))
 (segment (start 134.42 127.181) (end 132.08 124.841) (width 0.25) (layer F.Cu) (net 29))
 (segment (start 132.08 124.841) (end 132.08 115.57) (width 0.25) (layer F.Cu) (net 29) (status 20))
 (segment (start 128.09 106.5) (end 129.54 107.95) (width 0.25) (layer F.Cu) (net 33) (status 20))
 (segment (start 115.575 106.925) (end 116 106.5) (width 0.25) (layer F.Cu) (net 33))
 (segment (start 115.575 112.375) (end 115.575 106.925) (width 0.25) (layer F.Cu) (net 33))
 (segment (start 153.5 107.95) (end 148.84999 112.60001) (width 0.25) (layer F.Cu) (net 33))
 (segment (start 115.80001 112.60001) (end 115.575 112.375) (width 0.25) (layer F.Cu) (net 33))
 (segment (start 116 106.5) (end 128.09 106.5) (width 0.25) (layer F.Cu) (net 33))
 (segment (start 148.84999 112.60001) (end 115.80001 112.60001) (width 0.25) (layer F.Cu) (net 33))
 (segment (start 154.94 107.95) (end 153.5 107.95) (width 0.25) (layer F.Cu) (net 33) (status 10))
 (segment (start 166.37 107.95) (end 167.65 106.67) (width 0.25) (layer F.Cu) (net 34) (status 10))
 (segment (start 167.65 100.636238) (end 167.575 100.561238) (width 0.25) (layer F.Cu) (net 34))
 (segment (start 167.65 106.67) (end 167.65 100.636238) (width 0.25) (layer F.Cu) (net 34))
 (segment (start 167.575 100.561238) (end 167.575 99.95) (width 0.25) (layer F.Cu) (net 34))
 (segment (start 167.575 99.95) (end 167.325 99.7) (width 0.25) (layer F.Cu) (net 34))
 (segment (start 155.866238 99.7) (end 155.791238 99.775) (width 0.25) (layer F.Cu) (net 34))
 (segment (start 167.325 99.7) (end 155.866238 99.7) (width 0.25) (layer F.Cu) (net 34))
 (segment (start 155.791238 99.775) (end 155.3 99.775) (width 0.25) (layer F.Cu) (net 34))
 (segment (start 154.95 100.125) (end 154.95 101.58859) (width 0.25) (layer F.Cu) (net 34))
 (segment (start 155.3 99.775) (end 154.95 100.125) (width 0.25) (layer F.Cu) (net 34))
 (segment (start 154.95 101.58859) (end 149.86359 106.675) (width 0.25) (layer F.Cu) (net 34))
 (segment (start 133.355 106.675) (end 132.08 107.95) (width 0.25) (layer F.Cu) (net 34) (status 20))
 (segment (start 149.86359 106.675) (end 133.355 106.675) (width 0.25) (layer F.Cu) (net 34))
 (segment (start 136.398 90.932) (end 134.62 92.71) (width 0.25) (layer B.Cu) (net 6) (status 20))
 (segment (start 138.938 90.932) (end 136.398 90.932) (width 0.25) (layer B.Cu) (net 6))
 (segment (start 139.065 91.059) (end 138.938 90.932) (width 0.25) (layer B.Cu) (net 6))
 (segment (start 139.065 109.3) (end 139.065 91.059) (width 0.25) (layer B.Cu) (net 6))
 (segment (start 147.28 117.515) (end 139.065 109.3) (width 0.25) (layer B.Cu) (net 6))
 (segment (start 147.28 118.84) (end 147.28 117.515) (width 0.25) (layer B.Cu) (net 6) (status 10))
 (segment (start 119 112.15) (end 116.84 109.99) (width 0.25) (layer F.Cu) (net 8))
 (segment (start 156.037 104.013) (end 147.9 112.15) (width 0.25) (layer F.Cu) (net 8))
 (segment (start 116.84 109.99) (end 116.84 107.95) (width 0.25) (layer F.Cu) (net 8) (status 20))
 (segment (start 147.9 112.15) (end 119 112.15) (width 0.25) (layer F.Cu) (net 8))
 (segment (start 163.322 104.013) (end 156.037 104.013) (width 0.25) (layer F.Cu) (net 8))
 (segment (start 166.37 100.965) (end 163.322 104.013) (width 0.25) (layer F.Cu) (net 8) (status 10))
 (segment (start 163.068001 101.726999) (end 163.83 100.965) (width 0.25) (layer F.Cu) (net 9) (status 20))
 (segment (start 163.068 103.124) (end 163.068001 101.726999) (width 0.25) (layer F.Cu) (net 9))
 (segment (start 156.083 103.124) (end 163.068 103.124) (width 0.25) (layer F.Cu) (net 9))
 (segment (start 119.38 111.633) (end 147.574 111.633) (width 0.25) (layer F.Cu) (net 9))
 (segment (start 119.38 107.95) (end 119.38 111.633) (width 0.25) (layer F.Cu) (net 9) (status 10))
 (segment (start 147.574 111.633) (end 156.083 103.124) (width 0.25) (layer F.Cu) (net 9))
 (segment (start 155.8966 102.2944) (end 155.956 102.235) (width 0.25) (layer F.Cu) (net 11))
 (segment (start 122.174 111.125) (end 147.44559 111.125) (width 0.25) (layer F.Cu) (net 11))
 (segment (start 155.8966 102.67399) (end 155.8966 102.2944) (width 0.25) (layer F.Cu) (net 11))
 (segment (start 157.48 102.235) (end 158.75 100.965) (width 0.25) (layer F.Cu) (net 11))
 (segment (start 147.44559 111.125) (end 155.8966 102.67399) (width 0.25) (layer F.Cu) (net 11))
 (segment (start 121.92 110.871) (end 122.174 111.125) (width 0.25) (layer F.Cu) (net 11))
 (segment (start 155.956 102.235) (end 157.48 102.235) (width 0.25) (layer F.Cu) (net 11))
 (segment (start 121.92 107.95) (end 121.92 110.871) (width 0.25) (layer F.Cu) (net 11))
 (segment (start 150.495 106.68) (end 156.21 100.965) (width 0.25) (layer F.Cu) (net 12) (status 20))
 (segment (start 124.46 107.95) (end 124.46 110.236) (width 0.25) (layer F.Cu) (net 12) (status 10))
 (segment (start 124.46 110.236) (end 146.939 110.236) (width 0.25) (layer F.Cu) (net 12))
 (segment (start 146.939 110.236) (end 150.495 106.68) (width 0.25) (layer F.Cu) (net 12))
 (segment (start 149.78 102.155) (end 148.59 100.965) (width 0.4) (layer B.Cu) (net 5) (status 20))
 (segment (start 149.78 118.84) (end 149.78 102.155) (width 0.4) (layer B.Cu) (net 5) (status 10))
 (segment (start 109.22 92.71) (end 109.22 93.853) (width 0.4) (layer B.Cu) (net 5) (status 10))
 (segment (start 109.22 93.853) (end 108.331 94.742) (width 0.4) (layer B.Cu) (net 5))
 (segment (start 108.331 94.742) (end 108.331 96.012) (width 0.4) (layer B.Cu) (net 5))
 (segment (start 108.331 96.012) (end 107.315 97.028) (width 0.4) (layer B.Cu) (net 5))
 (segment (start 107.315 97.028) (end 102.489 97.028) (width 0.4) (layer B.Cu) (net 5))
 (segment (start 102.489 97.028) (end 102.362 97.155) (width 0.4) (layer B.Cu) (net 5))
 (segment (start 102.362 111.252) (end 106.68 115.57) (width 0.4) (layer B.Cu) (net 5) (status 20))
 (segment (start 102.362 97.155) (end 102.362 111.252) (width 0.4) (layer B.Cu) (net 5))
 (segment (start 124.46 115.57) (end 123.317 115.57) (width 0.4) (layer B.Cu) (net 5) (status 10))
 (segment (start 123.317 115.57) (end 123.317 116.586) (width 0.4) (layer B.Cu) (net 5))
 (segment (start 123.317 116.586) (end 122.936 116.967) (width 0.4) (layer B.Cu) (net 5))
 (segment (start 108.077 116.967) (end 106.68 115.57) (width 0.4) (layer B.Cu) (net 5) (status 20))
 (segment (start 122.936 116.967) (end 108.077 116.967) (width 0.4) (layer B.Cu) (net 5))
 (segment (start 149.78 102.155) (end 150.034 102.155) (width 0.4) (layer B.Cu) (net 5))
 (segment (start 150.034 102.155) (end 150.495 102.616) (width 0.4) (layer B.Cu) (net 5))
 (segment (start 152.019 102.616) (end 153.67 100.965) (width 0.4) (layer B.Cu) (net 5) (status 20))
 (segment (start 150.495 102.616) (end 152.019 102.616) (width 0.4) (layer B.Cu) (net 5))
 (segment (start 153.67 100.965) (end 155.321 102.616) (width 0.4) (layer B.Cu) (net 5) (status 10))
 (segment (start 167.259 102.616) (end 168.91 100.965) (width 0.4) (layer B.Cu) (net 5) (status 20))
 (segment (start 155.321 102.616) (end 167.259 102.616) (width 0.4) (layer B.Cu) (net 5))
 (segment (start 124.46 115.57) (end 124.46 116.935) (width 0.4) (layer B.Cu) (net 5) (status 10))
 (segment (start 124.46 116.935) (end 125.2 117.675) (width 0.4) (layer B.Cu) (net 5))
 (segment (start 125.2 117.675) (end 140.375 117.675) (width 0.4) (layer B.Cu) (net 5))
 (segment (start 140.375 117.675) (end 144.45 121.75) (width 0.4) (layer B.Cu) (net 5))
 (segment (start 146.87 121.75) (end 149.78 118.84) (width 0.4) (layer B.Cu) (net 5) (status 20))
 (segment (start 144.45 121.75) (end 146.87 121.75) (width 0.4) (layer B.Cu) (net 5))
 (segment (start 153.67 83.185) (end 151.13 85.725) (width 0.25) (layer F.Cu) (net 1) (status 20))
 (segment (start 153.67 78.74) (end 153.67 83.185) (width 0.25) (layer F.Cu) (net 1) (status 10))
 (segment (start 156.21 83.185) (end 153.67 85.725) (width 0.25) (layer F.Cu) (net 2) (status 20))
 (segment (start 156.21 78.74) (end 156.21 83.185) (width 0.25) (layer F.Cu) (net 2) (status 10)))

